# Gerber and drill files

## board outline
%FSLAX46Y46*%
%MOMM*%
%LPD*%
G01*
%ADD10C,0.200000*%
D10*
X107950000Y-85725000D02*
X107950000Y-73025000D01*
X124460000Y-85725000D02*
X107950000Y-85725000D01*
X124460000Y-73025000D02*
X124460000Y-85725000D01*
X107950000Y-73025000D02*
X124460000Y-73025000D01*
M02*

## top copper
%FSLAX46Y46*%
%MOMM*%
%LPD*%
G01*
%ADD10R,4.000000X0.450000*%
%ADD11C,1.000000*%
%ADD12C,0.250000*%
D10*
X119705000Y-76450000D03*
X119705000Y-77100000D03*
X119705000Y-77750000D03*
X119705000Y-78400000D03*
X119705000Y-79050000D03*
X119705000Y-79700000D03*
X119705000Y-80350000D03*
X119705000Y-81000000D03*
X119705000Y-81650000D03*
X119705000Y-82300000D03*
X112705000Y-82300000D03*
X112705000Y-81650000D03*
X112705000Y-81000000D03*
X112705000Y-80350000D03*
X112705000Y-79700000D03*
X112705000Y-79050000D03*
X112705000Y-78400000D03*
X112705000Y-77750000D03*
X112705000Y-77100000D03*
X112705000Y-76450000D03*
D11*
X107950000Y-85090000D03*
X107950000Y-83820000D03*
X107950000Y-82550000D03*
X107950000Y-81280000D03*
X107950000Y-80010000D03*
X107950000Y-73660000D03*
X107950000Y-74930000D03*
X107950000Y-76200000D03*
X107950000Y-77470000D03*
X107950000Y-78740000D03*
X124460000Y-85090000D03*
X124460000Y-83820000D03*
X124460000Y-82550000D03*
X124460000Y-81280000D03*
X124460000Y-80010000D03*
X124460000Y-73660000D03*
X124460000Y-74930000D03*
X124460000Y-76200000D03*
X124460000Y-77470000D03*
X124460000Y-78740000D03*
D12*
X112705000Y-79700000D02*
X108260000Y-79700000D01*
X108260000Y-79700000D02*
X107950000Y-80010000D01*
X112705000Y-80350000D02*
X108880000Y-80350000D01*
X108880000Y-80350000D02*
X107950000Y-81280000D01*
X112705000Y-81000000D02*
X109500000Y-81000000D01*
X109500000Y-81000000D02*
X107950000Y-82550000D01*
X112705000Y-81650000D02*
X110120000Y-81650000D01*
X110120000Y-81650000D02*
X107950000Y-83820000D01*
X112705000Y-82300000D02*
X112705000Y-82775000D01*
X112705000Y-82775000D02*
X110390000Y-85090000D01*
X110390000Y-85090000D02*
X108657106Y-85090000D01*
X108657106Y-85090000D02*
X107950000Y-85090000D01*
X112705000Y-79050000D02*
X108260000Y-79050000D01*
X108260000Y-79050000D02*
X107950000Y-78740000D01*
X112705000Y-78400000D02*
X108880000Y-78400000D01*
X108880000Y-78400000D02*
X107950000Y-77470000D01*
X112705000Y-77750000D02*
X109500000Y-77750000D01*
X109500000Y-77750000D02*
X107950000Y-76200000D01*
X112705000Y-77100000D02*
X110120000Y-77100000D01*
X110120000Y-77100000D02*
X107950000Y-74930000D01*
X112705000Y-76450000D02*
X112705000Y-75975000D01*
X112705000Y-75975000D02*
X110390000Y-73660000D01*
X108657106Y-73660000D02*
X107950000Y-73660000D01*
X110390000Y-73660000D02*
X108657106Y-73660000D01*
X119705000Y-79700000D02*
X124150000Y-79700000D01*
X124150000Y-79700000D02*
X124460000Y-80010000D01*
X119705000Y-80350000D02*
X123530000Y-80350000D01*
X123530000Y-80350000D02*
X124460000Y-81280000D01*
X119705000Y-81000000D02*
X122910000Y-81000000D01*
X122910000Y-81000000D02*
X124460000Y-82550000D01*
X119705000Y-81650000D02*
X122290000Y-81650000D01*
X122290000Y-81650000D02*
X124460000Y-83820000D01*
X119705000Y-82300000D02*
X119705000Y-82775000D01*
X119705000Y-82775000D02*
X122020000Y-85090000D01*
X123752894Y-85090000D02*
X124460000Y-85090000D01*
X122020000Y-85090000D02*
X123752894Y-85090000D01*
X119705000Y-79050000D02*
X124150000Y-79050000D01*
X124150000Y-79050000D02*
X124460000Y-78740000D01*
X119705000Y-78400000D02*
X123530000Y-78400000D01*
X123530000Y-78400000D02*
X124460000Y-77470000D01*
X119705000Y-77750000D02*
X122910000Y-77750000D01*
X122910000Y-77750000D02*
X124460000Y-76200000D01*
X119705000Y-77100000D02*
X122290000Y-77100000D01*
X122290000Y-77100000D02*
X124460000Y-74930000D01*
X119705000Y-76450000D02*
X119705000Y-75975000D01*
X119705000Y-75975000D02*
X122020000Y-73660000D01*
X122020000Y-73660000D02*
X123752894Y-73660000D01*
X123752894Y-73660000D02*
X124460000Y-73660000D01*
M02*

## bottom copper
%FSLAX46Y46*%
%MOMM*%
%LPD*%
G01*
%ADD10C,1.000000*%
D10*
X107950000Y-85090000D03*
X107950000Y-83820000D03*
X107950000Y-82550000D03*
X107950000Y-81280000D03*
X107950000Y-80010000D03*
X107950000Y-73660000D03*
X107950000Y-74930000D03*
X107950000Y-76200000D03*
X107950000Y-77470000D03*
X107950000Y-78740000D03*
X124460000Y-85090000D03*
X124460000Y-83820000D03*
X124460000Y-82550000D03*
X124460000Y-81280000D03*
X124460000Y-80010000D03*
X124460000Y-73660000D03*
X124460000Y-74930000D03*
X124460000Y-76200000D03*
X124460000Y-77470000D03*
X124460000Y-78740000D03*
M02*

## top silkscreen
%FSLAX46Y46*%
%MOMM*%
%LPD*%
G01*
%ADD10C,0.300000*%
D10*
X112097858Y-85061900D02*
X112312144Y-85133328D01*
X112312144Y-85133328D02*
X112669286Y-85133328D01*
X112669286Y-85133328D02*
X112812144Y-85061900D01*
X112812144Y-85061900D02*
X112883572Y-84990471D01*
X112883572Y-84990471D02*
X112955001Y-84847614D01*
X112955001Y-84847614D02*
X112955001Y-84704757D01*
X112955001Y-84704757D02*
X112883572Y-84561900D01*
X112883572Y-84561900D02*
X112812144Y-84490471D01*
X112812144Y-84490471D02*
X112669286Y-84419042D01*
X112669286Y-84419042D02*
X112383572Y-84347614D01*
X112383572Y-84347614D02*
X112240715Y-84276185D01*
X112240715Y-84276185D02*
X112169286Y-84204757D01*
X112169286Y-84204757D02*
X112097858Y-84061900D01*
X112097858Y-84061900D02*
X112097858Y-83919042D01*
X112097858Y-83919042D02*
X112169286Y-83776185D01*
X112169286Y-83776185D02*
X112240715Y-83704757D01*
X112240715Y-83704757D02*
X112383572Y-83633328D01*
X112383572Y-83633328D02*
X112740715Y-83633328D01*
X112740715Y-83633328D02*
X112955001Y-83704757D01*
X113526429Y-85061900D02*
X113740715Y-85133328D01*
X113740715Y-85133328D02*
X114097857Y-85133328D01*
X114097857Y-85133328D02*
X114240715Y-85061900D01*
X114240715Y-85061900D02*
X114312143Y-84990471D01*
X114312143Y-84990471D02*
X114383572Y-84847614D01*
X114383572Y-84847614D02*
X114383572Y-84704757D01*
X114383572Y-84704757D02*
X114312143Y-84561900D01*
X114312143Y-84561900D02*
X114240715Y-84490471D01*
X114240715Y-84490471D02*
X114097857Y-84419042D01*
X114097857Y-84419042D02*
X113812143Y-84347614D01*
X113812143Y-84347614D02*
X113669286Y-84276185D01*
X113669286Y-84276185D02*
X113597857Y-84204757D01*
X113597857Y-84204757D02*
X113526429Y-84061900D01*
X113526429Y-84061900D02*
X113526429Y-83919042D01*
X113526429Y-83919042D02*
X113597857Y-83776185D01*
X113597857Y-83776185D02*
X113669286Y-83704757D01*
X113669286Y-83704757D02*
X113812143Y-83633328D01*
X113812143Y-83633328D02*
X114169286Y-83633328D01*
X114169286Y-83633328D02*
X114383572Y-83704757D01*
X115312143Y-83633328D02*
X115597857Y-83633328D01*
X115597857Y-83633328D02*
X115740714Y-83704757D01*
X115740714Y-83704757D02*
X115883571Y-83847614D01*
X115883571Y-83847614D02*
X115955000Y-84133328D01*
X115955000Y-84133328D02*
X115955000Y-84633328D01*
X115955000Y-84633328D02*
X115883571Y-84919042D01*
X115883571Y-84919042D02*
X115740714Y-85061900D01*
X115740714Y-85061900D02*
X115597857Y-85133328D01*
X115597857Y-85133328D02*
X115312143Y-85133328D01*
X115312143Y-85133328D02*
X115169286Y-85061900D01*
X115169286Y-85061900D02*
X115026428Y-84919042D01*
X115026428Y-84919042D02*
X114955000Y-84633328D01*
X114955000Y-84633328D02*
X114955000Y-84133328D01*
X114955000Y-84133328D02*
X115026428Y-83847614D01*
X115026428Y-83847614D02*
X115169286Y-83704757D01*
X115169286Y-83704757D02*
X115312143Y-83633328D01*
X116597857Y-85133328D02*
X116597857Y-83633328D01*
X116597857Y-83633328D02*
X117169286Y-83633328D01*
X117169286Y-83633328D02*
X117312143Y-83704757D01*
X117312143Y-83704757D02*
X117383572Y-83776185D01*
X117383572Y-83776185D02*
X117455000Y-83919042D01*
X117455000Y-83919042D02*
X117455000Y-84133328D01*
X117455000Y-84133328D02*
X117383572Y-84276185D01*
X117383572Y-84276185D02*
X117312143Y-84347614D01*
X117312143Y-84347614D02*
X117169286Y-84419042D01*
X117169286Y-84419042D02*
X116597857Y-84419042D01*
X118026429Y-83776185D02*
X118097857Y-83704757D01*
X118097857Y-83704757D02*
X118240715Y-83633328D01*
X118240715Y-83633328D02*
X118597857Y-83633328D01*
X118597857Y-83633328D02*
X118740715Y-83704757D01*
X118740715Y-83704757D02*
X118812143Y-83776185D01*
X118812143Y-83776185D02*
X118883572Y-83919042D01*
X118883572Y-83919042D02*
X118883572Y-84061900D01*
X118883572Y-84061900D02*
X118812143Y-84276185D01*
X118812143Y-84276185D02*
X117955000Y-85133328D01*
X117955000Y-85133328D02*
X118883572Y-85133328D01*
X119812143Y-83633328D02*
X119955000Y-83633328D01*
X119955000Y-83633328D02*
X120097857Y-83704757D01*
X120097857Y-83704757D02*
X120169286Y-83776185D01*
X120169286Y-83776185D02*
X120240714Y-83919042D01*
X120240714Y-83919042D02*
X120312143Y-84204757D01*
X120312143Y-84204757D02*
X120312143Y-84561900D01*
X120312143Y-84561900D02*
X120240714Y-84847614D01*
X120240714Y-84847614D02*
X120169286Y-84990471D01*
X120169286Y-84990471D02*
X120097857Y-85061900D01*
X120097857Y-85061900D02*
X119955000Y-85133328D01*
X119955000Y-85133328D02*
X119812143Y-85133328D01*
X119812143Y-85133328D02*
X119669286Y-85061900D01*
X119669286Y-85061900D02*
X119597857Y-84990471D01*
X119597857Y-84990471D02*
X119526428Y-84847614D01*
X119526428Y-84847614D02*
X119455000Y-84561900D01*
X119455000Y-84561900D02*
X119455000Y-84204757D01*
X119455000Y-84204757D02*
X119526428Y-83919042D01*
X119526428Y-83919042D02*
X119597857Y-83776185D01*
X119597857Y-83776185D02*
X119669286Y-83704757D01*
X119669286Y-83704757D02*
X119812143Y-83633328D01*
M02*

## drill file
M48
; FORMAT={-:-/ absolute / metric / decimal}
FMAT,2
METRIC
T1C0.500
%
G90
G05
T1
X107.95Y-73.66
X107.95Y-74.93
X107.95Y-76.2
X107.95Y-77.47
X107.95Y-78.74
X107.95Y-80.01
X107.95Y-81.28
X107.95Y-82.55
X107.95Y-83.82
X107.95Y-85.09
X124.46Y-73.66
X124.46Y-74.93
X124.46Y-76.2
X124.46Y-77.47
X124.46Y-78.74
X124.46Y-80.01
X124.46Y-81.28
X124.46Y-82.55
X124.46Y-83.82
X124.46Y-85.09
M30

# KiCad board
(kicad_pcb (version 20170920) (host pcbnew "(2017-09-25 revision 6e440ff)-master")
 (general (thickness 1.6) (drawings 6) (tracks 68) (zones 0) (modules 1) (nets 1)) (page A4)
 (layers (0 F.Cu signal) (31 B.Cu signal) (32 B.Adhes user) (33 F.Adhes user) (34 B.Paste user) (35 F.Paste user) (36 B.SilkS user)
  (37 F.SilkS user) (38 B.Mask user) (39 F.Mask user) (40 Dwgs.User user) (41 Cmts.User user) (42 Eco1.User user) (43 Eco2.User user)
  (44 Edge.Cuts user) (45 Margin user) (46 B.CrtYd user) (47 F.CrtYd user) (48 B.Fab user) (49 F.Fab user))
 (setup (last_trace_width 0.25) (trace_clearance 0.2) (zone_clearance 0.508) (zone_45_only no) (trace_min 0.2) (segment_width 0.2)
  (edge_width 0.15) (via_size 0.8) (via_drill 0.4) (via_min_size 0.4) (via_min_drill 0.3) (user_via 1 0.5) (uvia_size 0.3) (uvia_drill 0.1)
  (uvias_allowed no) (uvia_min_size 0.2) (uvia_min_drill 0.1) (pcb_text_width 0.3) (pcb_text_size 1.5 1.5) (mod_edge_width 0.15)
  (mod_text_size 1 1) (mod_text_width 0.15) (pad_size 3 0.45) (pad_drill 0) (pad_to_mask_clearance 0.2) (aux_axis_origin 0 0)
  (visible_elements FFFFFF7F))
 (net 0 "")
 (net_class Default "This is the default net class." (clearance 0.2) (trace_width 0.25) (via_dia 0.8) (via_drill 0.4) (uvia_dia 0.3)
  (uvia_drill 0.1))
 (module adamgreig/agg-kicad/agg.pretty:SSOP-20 (layer F.Cu) (at 116.205 79.375)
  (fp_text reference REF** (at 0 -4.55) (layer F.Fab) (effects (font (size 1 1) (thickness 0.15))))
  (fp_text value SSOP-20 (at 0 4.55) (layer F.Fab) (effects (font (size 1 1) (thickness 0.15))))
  (pad 20 smd rect (at 3.5 -2.925) (size 4 0.45) (layers F.Cu F.Paste F.Mask))
  (pad 19 smd rect (at 3.5 -2.275) (size 4 0.45) (layers F.Cu F.Paste F.Mask))
  (pad 18 smd rect (at 3.5 -1.625) (size 4 0.45) (layers F.Cu F.Paste F.Mask))
  (pad 17 smd rect (at 3.5 -0.975) (size 4 0.45) (layers F.Cu F.Paste F.Mask))
  (pad 16 smd rect (at 3.5 -0.325) (size 4 0.45) (layers F.Cu F.Paste F.Mask))
  (pad 15 smd rect (at 3.5 0.325) (size 4 0.45) (layers F.Cu F.Paste F.Mask))
  (pad 14 smd rect (at 3.5 0.975) (size 4 0.45) (layers F.Cu F.Paste F.Mask))
  (pad 13 smd rect (at 3.5 1.625) (size 4 0.45) (layers F.Cu F.Paste F.Mask))
  (pad 12 smd rect (at 3.5 2.275) (size 4 0.45) (layers F.Cu F.Paste F.Mask))
  (pad 11 smd rect (at 3.5 2.925) (size 4 0.45) (layers F.Cu F.Paste F.Mask))
  (pad 10 smd rect (at -3.5 2.925) (size 4 0.45) (layers F.Cu F.Paste F.Mask))
  (pad 9 smd rect (at -3.5 2.275) (size 4 0.45) (layers F.Cu F.Paste F.Mask))
  (pad 8 smd rect (at -3.5 1.625) (size 4 0.45) (layers F.Cu F.Paste F.Mask))
  (pad 7 smd rect (at -3.5 0.975) (size 4 0.45) (layers F.Cu F.Paste F.Mask))
  (pad 6 smd rect (at -3.5 0.325) (size 4 0.45) (layers F.Cu F.Paste F.Mask))
  (pad 5 smd rect (at -3.5 -0.325) (size 4 0.45) (layers F.Cu F.Paste F.Mask))
  (pad 4 smd rect (at -3.5 -0.975) (size 4 0.45) (layers F.Cu F.Paste F.Mask))
  (pad 3 smd rect (at -3.5 -1.625) (size 4 0.45) (layers F.Cu F.Paste F.Mask))
  (pad 2 smd rect (at -3.5 -2.275) (size 4 0.45) (layers F.Cu F.Paste F.Mask))
  (pad 1 smd rect (at -3.5 -2.925) (size 4 0.45) (layers F.Cu F.Paste F.Mask)))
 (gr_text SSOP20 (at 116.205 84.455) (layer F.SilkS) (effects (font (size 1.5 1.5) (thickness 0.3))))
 (gr_line (start 107.95 85.725) (end 107.95 73.025) (layer Edge.Cuts) (width 0.2))
 (gr_line (start 124.46 85.725) (end 107.95 85.725) (layer Edge.Cuts) (width 0.2))
 (gr_line (start 124.46 73.025) (end 124.46 85.725) (layer Edge.Cuts) (width 0.2))
 (gr_line (start 107.95 73.025) (end 124.46 73.025) (layer Edge.Cuts) (width 0.2))
 (segment (start 112.705 79.7) (end 108.26 79.7) (width 0.25) (layer F.Cu) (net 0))
 (segment (start 108.26 79.7) (end 107.95 80.01) (width 0.25) (layer F.Cu) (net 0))
 (segment (start 112.705 80.35) (end 108.88 80.35) (width 0.25) (layer F.Cu) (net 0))
 (segment (start 108.88 80.35) (end 107.95 81.28) (width 0.25) (layer F.Cu) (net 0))
 (segment (start 112.705 81) (end 109.5 81) (width 0.25) (layer F.Cu) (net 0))
 (segment (start 109.5 81) (end 107.95 82.55) (width 0.25) (layer F.Cu) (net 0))
 (segment (start 112.705 81.65) (end 110.12 81.65) (width 0.25) (layer F.Cu) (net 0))
 (segment (start 110.12 81.65) (end 107.95 83.82) (width 0.25) (layer F.Cu) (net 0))
 (segment (start 112.705 82.3) (end 112.705 82.775) (width 0.25) (layer F.Cu) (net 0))
 (segment (start 112.705 82.775) (end 110.39 85.09) (width 0.25) (layer F.Cu) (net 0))
 (segment (start 110.39 85.09) (end 108.657106 85.09) (width 0.25) (layer F.Cu) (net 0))
 (segment (start 108.657106 85.09) (end 107.95 85.09) (width 0.25) (layer F.Cu) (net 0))
 (segment (start 112.705 79.05) (end 108.26 79.05) (width 0.25) (layer F.Cu) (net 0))
 (segment (start 108.26 79.05) (end 107.95 78.74) (width 0.25) (layer F.Cu) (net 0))
 (segment (start 112.705 78.4) (end 108.88 78.4) (width 0.25) (layer F.Cu) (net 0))
 (segment (start 108.88 78.4) (end 107.95 77.47) (width 0.25) (layer F.Cu) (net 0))
 (segment (start 112.705 77.75) (end 109.5 77.75) (width 0.25) (layer F.Cu) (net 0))
 (segment (start 109.5 77.75) (end 107.95 76.2) (width 0.25) (layer F.Cu) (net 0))
 (segment (start 112.705 77.1) (end 110.12 77.1) (width 0.25) (layer F.Cu) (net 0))
 (segment (start 110.12 77.1) (end 107.95 74.93) (width 0.25) (layer F.Cu) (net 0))
 (segment (start 112.705 76.45) (end 112.705 75.975) (width 0.25) (layer F.Cu) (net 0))
 (segment (start 112.705 75.975) (end 110.39 73.66) (width 0.25) (layer F.Cu) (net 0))
 (segment (start 108.657106 73.66) (end 107.95 73.66) (width 0.25) (layer F.Cu) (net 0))
 (segment (start 110.39 73.66) (end 108.657106 73.66) (width 0.25) (layer F.Cu) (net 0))
 (segment (start 119.705 79.7) (end 124.15 79.7) (width 0.25) (layer F.Cu) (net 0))
 (segment (start 124.15 79.7) (end 124.46 80.01) (width 0.25) (layer F.Cu) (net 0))
 (segment (start 119.705 80.35) (end 123.53 80.35) (width 0.25) (layer F.Cu) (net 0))
 (segment (start 123.53 80.35) (end 124.46 81.28) (width 0.25) (layer F.Cu) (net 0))
 (segment (start 119.705 81) (end 122.91 81) (width 0.25) (layer F.Cu) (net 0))
 (segment (start 122.91 81) (end 124.46 82.55) (width 0.25) (layer F.Cu) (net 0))
 (segment (start 119.705 81.65) (end 122.29 81.65) (width 0.25) (layer F.Cu) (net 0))
 (segment (start 122.29 81.65) (end 124.46 83.82) (width 0.25) (layer F.Cu) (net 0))
 (segment (start 119.705 82.3) (end 119.705 82.775) (width 0.25) (layer F.Cu) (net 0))
 (segment (start 119.705 82.775) (end 122.02 85.09) (width 0.25) (layer F.Cu) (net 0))
 (segment (start 123.752894 85.09) (end 124.46 85.09) (width 0.25) (layer F.Cu) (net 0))
 (segment (start 122.02 85.09) (end 123.752894 85.09) (width 0.25) (layer F.Cu) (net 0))
 (segment (start 119.705 79.05) (end 124.15 79.05) (width 0.25) (layer F.Cu) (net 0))
 (segment (start 124.15 79.05) (end 124.46 78.74) (width 0.25) (layer F.Cu) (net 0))
 (segment (start 119.705 78.4) (end 123.53 78.4) (width 0.25) (layer F.Cu) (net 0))
 (segment (start 123.53 78.4) (end 124.46 77.47) (width 0.25) (layer F.Cu) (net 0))
 (segment (start 119.705 77.75) (end 122.91 77.75) (width 0.25) (layer F.Cu) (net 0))
 (segment (start 122.91 77.75) (end 124.46 76.2) (width 0.25) (layer F.Cu) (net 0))
 (segment (start 119.705 77.1) (end 122.29 77.1) (width 0.25) (layer F.Cu) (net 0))
 (segment (start 122.29 77.1) (end 124.46 74.93) (width 0.25) (layer F.Cu) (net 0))
 (segment (start 119.705 76.45) (end 119.705 75.975) (width 0.25) (layer F.Cu) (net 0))
 (segment (start 119.705 75.975) (end 122.02 73.66) (width 0.25) (layer F.Cu) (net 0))
 (segment (start 122.02 73.66) (end 123.752894 73.66) (width 0.25) (layer F.Cu) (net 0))
 (segment (start 123.752894 73.66) (end 124.46 73.66) (width 0.25) (layer F.Cu) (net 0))
 (via (at 107.95 85.09) (size 1) (drill 0.5) (layers F.Cu B.Cu) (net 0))
 (via (at 107.95 83.82) (size 1) (drill 0.5) (layers F.Cu B.Cu) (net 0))
 (via (at 107.95 82.55) (size 1) (drill 0.5) (layers F.Cu B.Cu) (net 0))
 (via (at 107.95 81.28) (size 1) (drill 0.5) (layers F.Cu B.Cu) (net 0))
 (via (at 107.95 80.01) (size 1) (drill 0.5) (layers F.Cu B.Cu) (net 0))
 (via (at 107.95 73.66) (size 1) (drill 0.5) (layers F.Cu B.Cu) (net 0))
 (via (at 107.95 74.93) (size 1) (drill 0.5) (layers F.Cu B.Cu) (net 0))
 (via (at 107.95 76.2) (size 1) (drill 0.5) (layers F.Cu B.Cu) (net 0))
 (via (at 107.95 77.47) (size 1) (drill 0.5) (layers F.Cu B.Cu) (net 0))
 (via (at 107.95 78.74) (size 1) (drill 0.5) (layers F.Cu B.Cu) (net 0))
 (via (at 124.46 85.09) (size 1) (drill 0.5) (layers F.Cu B.Cu) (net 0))
 (via (at 124.46 83.82) (size 1) (drill 0.5) (layers F.Cu B.Cu) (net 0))
 (via (at 124.46 82.55) (size 1) (drill 0.5) (layers F.Cu B.Cu) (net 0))
 (via (at 124.46 81.28) (size 1) (drill 0.5) (layers F.Cu B.Cu) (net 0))
 (via (at 124.46 80.01) (size 1) (drill 0.5) (layers F.Cu B.Cu) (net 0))
 (via (at 124.46 73.66) (size 1) (drill 0.5) (layers F.Cu B.Cu) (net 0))
 (via (at 124.46 74.93) (size 1) (drill 0.5) (layers F.Cu B.Cu) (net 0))
 (via (at 124.46 76.2) (size 1) (drill 0.5) (layers F.Cu B.Cu) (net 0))
 (via (at 124.46 77.47) (size 1) (drill 0.5) (layers F.Cu B.Cu) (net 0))
 (via (at 124.46 78.74) (size 1) (drill 0.5) (layers F.Cu B.Cu) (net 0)))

